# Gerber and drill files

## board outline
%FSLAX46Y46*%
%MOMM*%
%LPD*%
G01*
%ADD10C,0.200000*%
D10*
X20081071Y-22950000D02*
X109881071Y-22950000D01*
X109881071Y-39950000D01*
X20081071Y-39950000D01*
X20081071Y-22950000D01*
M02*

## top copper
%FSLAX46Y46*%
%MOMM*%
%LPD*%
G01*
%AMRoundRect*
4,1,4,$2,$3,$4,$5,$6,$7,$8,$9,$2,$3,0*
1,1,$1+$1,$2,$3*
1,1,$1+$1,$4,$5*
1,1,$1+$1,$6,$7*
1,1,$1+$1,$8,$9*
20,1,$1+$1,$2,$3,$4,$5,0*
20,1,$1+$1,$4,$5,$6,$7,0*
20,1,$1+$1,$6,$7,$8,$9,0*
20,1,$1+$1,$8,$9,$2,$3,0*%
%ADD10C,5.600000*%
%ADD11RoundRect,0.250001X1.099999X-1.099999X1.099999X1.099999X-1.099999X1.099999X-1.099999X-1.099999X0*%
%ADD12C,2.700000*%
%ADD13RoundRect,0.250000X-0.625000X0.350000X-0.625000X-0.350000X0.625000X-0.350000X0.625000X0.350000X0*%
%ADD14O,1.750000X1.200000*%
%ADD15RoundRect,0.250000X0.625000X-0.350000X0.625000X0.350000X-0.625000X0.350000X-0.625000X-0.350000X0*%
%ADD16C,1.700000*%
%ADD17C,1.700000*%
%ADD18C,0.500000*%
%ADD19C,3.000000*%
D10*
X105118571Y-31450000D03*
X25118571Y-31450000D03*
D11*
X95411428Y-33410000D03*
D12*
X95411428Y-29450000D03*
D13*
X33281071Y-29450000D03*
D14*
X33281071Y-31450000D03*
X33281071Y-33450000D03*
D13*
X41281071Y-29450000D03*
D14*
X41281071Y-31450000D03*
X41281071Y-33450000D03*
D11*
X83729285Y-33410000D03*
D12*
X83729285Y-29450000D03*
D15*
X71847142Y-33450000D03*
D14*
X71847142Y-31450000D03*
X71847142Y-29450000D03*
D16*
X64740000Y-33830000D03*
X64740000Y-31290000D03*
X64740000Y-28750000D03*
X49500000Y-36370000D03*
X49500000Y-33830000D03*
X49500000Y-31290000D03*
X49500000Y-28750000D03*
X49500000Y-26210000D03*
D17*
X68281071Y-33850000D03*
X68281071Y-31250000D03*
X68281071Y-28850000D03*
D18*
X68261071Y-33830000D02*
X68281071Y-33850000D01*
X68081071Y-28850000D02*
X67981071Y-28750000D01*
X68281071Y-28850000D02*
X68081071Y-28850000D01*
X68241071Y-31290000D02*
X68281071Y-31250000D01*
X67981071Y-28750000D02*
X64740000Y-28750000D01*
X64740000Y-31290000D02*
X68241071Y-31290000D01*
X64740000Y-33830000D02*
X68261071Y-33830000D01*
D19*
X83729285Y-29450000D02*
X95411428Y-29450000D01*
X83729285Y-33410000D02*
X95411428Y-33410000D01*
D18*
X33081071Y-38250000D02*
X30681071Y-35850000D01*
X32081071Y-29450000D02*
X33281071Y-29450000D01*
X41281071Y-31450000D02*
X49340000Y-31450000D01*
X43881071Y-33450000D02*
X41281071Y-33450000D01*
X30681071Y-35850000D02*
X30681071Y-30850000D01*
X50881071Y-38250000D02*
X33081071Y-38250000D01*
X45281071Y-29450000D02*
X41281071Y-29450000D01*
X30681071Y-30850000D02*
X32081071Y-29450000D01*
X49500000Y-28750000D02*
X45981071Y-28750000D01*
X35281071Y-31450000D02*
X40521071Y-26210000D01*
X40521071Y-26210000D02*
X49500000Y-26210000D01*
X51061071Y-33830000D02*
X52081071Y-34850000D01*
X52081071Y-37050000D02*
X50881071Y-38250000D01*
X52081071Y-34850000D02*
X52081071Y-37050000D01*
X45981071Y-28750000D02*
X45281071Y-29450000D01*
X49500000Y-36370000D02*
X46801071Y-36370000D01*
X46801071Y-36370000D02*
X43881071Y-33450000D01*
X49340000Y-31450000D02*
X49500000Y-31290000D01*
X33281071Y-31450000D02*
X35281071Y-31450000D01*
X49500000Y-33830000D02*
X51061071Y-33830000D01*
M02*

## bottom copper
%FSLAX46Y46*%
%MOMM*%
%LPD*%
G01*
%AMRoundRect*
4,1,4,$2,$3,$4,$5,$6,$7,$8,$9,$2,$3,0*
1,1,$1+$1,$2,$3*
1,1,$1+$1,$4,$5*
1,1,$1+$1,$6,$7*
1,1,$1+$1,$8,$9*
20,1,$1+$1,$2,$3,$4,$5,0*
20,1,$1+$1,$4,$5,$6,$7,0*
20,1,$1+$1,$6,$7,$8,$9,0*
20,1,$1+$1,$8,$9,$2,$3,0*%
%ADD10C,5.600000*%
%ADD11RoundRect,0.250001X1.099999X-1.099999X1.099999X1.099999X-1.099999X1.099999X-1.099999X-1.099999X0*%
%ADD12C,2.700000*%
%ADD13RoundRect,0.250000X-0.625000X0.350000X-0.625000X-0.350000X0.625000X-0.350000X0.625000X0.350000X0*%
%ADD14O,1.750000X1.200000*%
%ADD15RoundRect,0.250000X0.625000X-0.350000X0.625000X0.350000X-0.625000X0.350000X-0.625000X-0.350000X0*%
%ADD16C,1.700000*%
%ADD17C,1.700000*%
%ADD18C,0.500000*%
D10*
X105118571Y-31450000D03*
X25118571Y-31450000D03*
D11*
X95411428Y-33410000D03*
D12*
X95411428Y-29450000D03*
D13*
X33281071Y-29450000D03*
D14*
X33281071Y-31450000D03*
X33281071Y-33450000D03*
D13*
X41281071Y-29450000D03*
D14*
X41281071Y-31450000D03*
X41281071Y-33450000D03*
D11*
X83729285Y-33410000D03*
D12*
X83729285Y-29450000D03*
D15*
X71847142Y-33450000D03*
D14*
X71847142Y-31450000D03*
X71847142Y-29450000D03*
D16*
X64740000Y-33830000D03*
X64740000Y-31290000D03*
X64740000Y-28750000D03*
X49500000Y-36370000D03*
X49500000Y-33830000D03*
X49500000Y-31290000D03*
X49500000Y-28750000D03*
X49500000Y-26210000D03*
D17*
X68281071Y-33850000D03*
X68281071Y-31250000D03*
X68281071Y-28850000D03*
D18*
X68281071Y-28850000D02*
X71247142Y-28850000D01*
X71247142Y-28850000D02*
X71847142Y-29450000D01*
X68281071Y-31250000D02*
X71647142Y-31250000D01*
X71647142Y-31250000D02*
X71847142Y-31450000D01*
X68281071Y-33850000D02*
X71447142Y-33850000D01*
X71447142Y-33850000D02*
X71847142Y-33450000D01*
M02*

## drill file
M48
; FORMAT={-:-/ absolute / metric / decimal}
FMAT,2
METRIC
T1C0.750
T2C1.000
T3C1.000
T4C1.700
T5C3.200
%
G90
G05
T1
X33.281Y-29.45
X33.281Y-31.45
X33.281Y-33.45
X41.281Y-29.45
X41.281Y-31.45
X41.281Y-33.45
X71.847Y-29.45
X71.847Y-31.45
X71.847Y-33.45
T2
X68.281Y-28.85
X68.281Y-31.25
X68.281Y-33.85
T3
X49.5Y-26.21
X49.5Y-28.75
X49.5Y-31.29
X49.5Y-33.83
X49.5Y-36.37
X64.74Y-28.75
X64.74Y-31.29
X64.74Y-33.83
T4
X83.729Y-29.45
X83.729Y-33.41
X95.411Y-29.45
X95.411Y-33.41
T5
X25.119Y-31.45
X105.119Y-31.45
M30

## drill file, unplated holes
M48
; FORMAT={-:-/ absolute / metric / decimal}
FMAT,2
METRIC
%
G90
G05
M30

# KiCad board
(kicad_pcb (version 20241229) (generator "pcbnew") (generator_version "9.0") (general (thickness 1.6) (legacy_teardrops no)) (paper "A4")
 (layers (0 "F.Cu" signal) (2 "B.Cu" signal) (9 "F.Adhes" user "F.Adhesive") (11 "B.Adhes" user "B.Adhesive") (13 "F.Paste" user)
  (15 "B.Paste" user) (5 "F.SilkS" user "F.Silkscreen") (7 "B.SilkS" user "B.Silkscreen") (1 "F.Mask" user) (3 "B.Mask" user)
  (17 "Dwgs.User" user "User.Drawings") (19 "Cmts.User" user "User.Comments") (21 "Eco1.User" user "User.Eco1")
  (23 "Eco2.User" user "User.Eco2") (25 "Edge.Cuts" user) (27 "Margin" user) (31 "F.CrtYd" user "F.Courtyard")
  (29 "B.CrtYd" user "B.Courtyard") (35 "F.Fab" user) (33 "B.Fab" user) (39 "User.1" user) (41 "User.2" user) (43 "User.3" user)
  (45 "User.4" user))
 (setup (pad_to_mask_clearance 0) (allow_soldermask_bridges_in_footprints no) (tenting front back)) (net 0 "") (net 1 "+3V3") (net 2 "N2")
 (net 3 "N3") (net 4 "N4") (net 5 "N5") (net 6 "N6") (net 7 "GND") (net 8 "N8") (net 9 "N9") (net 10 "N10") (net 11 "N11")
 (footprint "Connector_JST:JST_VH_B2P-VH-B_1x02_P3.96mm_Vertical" (layer "F.Cu") (at 95.411428 33.41 90)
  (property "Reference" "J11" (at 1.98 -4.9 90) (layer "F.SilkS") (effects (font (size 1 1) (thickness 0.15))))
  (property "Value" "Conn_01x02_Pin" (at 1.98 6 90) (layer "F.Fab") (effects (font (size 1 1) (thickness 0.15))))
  (pad "1" thru_hole roundrect (at 0 0 90) (size 2.7 2.7) (drill 1.7) (layers "*.Cu" "*.Mask") (remove_unused_layers no)
   (roundrect_rratio 0.092593) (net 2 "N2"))
  (pad "2" thru_hole circle (at 3.96 0 90) (size 2.7 2.7) (drill 1.7) (layers "*.Cu" "*.Mask") (remove_unused_layers no) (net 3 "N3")))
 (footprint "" (layer "F.Cu") (at 105.118571 31.45)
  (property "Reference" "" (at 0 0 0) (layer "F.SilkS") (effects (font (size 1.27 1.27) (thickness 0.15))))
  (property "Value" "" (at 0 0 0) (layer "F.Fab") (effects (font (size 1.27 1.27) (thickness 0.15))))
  (pad "1" thru_hole circle (at 0 0) (size 5.6 5.6) (drill 3.2) (layers "*.Cu" "*.Mask") (remove_unused_layers no) (zone_connect 2)))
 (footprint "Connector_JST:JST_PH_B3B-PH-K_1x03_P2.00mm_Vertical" (layer "F.Cu") (at 71.847142 33.45 90)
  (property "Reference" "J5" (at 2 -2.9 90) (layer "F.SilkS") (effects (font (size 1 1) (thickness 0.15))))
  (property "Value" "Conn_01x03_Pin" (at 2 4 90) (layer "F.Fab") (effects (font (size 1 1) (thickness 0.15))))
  (pad "1" thru_hole roundrect (at 0 0 90) (size 1.2 1.75) (drill 0.75) (layers "*.Cu" "*.Mask") (remove_unused_layers no)
   (roundrect_rratio 0.208333) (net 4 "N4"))
  (pad "2" thru_hole oval (at 2 0 90) (size 1.2 1.75) (drill 0.75) (layers "*.Cu" "*.Mask") (remove_unused_layers no) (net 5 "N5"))
  (pad "3" thru_hole oval (at 4 0 90) (size 1.2 1.75) (drill 0.75) (layers "*.Cu" "*.Mask") (remove_unused_layers no) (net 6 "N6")))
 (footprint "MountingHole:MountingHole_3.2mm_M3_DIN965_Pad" (layer "F.Cu") (at 25.118571 31.45)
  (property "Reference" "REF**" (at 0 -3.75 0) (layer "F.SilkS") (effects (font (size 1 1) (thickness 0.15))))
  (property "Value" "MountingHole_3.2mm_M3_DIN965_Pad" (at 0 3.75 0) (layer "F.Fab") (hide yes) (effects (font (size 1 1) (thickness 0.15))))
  (pad "1" thru_hole circle (at 0 0) (size 5.6 5.6) (drill 3.2) (layers "*.Cu" "*.Mask") (remove_unused_layers no) (zone_connect 2)))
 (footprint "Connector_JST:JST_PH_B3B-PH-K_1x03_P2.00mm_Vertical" (layer "B.Cu") (at 33.281071 29.45 -90)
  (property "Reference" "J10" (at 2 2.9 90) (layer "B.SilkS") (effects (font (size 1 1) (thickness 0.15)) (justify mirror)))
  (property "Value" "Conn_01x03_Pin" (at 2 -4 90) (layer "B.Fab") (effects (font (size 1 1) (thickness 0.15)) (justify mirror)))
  (pad "1" thru_hole roundrect (at 0 0 270) (size 1.2 1.75) (drill 0.75) (layers "*.Cu" "*.Mask") (remove_unused_layers no)
   (roundrect_rratio 0.208333) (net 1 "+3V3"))
  (pad "2" thru_hole oval (at 2 0 270) (size 1.2 1.75) (drill 0.75) (layers "*.Cu" "*.Mask") (remove_unused_layers no) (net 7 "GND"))
  (pad "3" thru_hole oval (at 4 0 270) (size 1.2 1.75) (drill 0.75) (layers "*.Cu" "*.Mask") (remove_unused_layers no) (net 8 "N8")))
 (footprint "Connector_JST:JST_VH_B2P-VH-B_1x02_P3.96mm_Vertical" (layer "B.Cu") (at 83.729285 33.41 90)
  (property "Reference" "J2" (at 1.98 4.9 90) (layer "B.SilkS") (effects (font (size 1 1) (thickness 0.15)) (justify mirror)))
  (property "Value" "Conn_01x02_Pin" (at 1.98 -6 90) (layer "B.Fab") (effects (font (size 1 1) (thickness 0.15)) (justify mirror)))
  (pad "1" thru_hole roundrect (at 0 0 90) (size 2.7 2.7) (drill 1.7) (layers "*.Cu" "*.Mask") (remove_unused_layers no)
   (roundrect_rratio 0.092593) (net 2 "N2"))
  (pad "2" thru_hole circle (at 3.96 0 90) (size 2.7 2.7) (drill 1.7) (layers "*.Cu" "*.Mask") (remove_unused_layers no) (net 3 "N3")))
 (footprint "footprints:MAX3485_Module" (layer "B.Cu") (at 60.74 26.79 90)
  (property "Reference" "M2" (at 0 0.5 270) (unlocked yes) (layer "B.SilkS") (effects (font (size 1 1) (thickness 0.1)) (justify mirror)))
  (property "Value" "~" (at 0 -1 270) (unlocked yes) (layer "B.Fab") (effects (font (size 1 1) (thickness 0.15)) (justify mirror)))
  (pad "1" thru_hole circle (at -7.04 4 90) (size 1.7 1.7) (drill 1) (layers "*.Cu" "*.Mask") (remove_unused_layers no) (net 4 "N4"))
  (pad "2" thru_hole circle (at -4.5 4 90) (size 1.7 1.7) (drill 1) (layers "*.Cu" "*.Mask") (remove_unused_layers no) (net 5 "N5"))
  (pad "3" thru_hole circle (at -1.96 4 90) (size 1.7 1.7) (drill 1) (layers "*.Cu" "*.Mask") (remove_unused_layers no) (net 6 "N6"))
  (pad "4" thru_hole circle (at -9.58 -11.24 90) (size 1.7 1.7) (drill 1) (layers "*.Cu" "*.Mask") (remove_unused_layers no) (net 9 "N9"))
  (pad "5" thru_hole circle (at -7.04 -11.24 90) (size 1.7 1.7) (drill 1) (layers "*.Cu" "*.Mask") (remove_unused_layers no) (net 1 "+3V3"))
  (pad "6" thru_hole circle (at -4.5 -11.24 90) (size 1.7 1.7) (drill 1) (layers "*.Cu" "*.Mask") (remove_unused_layers no) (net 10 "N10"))
  (pad "7" thru_hole circle (at -1.96 -11.24 90) (size 1.7 1.7) (drill 1) (layers "*.Cu" "*.Mask") (remove_unused_layers no) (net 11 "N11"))
  (pad "8" thru_hole circle (at 0.58 -11.24 90) (size 1.7 1.7) (drill 1) (layers "*.Cu" "*.Mask") (remove_unused_layers no) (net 7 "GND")))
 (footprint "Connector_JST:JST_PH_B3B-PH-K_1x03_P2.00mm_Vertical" (layer "B.Cu") (at 41.281071 29.45 -90)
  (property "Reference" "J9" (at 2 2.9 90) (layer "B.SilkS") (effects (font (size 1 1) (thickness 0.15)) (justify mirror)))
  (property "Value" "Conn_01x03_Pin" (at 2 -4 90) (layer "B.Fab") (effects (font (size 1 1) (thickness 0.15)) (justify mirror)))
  (pad "1" thru_hole roundrect (at 0 0 270) (size 1.2 1.75) (drill 0.75) (layers "*.Cu" "*.Mask") (remove_unused_layers no)
   (roundrect_rratio 0.208333) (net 11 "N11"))
  (pad "2" thru_hole oval (at 2 0 270) (size 1.2 1.75) (drill 0.75) (layers "*.Cu" "*.Mask") (remove_unused_layers no) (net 10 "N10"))
  (pad "3" thru_hole oval (at 4 0 270) (size 1.2 1.75) (drill 0.75) (layers "*.Cu" "*.Mask") (remove_unused_layers no) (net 9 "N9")))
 (gr_rect (start 20.081071 22.95) (end 109.881071 39.95) (stroke (width 0.2) (type solid)) (fill no) (layer "Edge.Cuts"))
 (segment (start 52.081071 37.05) (end 50.881071 38.25) (width 0.5) (layer "F.Cu") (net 1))
 (segment (start 51.061071 33.83) (end 52.081071 34.85) (width 0.5) (layer "F.Cu") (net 1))
 (segment (start 32.081071 29.45) (end 33.281071 29.45) (width 0.5) (layer "F.Cu") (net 1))
 (segment (start 30.681071 30.85) (end 32.081071 29.45) (width 0.5) (layer "F.Cu") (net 1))
 (segment (start 30.681071 35.85) (end 30.681071 30.85) (width 0.5) (layer "F.Cu") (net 1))
 (segment (start 52.081071 34.85) (end 52.081071 37.05) (width 0.5) (layer "F.Cu") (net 1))
 (segment (start 33.081071 38.25) (end 30.681071 35.85) (width 0.5) (layer "F.Cu") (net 1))
 (segment (start 49.5 33.83) (end 51.061071 33.83) (width 0.5) (layer "F.Cu") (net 1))
 (segment (start 50.881071 38.25) (end 33.081071 38.25) (width 0.5) (layer "F.Cu") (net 1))
 (segment (start 40.521071 26.21) (end 49.5 26.21) (width 0.5) (layer "F.Cu") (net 7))
 (segment (start 35.281071 31.45) (end 40.521071 26.21) (width 0.5) (layer "F.Cu") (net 7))
 (segment (start 33.281071 31.45) (end 35.281071 31.45) (width 0.5) (layer "F.Cu") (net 7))
 (segment (start 41.281071 31.45) (end 49.34 31.45) (width 0.5) (layer "F.Cu") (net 10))
 (segment (start 49.34 31.45) (end 49.5 31.29) (width 0.5) (layer "F.Cu") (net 10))
 (segment (start 43.881071 33.45) (end 41.281071 33.45) (width 0.5) (layer "F.Cu") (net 9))
 (segment (start 46.801071 36.37) (end 43.881071 33.45) (width 0.5) (layer "F.Cu") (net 9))
 (segment (start 49.5 36.37) (end 46.801071 36.37) (width 0.5) (layer "F.Cu") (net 9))
 (segment (start 45.981071 28.75) (end 45.281071 29.45) (width 0.5) (layer "F.Cu") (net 11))
 (segment (start 49.5 28.75) (end 45.981071 28.75) (width 0.5) (layer "F.Cu") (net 11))
 (segment (start 45.281071 29.45) (end 41.281071 29.45) (width 0.5) (layer "F.Cu") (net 11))
 (segment (start 67.981071 28.75) (end 64.74 28.75) (width 0.5) (layer "F.Cu") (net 6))
 (segment (start 68.081071 28.85) (end 67.981071 28.75) (width 0.5) (layer "F.Cu") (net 6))
 (segment (start 68.281071 28.85) (end 68.081071 28.85) (width 0.5) (layer "F.Cu") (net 6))
 (via (at 68.281071 28.85) (size 1.7) (drill 1) (layers "F.Cu" "B.Cu") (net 6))
 (segment (start 68.281071 28.85) (end 71.247142 28.85) (width 0.5) (layer "B.Cu") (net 6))
 (segment (start 71.247142 28.85) (end 71.847142 29.45) (width 0.5) (layer "B.Cu") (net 6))
 (segment (start 68.241071 31.29) (end 68.281071 31.25) (width 0.5) (layer "F.Cu") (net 5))
 (segment (start 64.74 31.29) (end 68.241071 31.29) (width 0.5) (layer "F.Cu") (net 5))
 (via (at 68.281071 31.25) (size 1.7) (drill 1) (layers "F.Cu" "B.Cu") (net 5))
 (segment (start 71.647142 31.25) (end 71.847142 31.45) (width 0.5) (layer "B.Cu") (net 5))
 (segment (start 68.281071 31.25) (end 71.647142 31.25) (width 0.5) (layer "B.Cu") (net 5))
 (segment (start 68.261071 33.83) (end 68.281071 33.85) (width 0.5) (layer "F.Cu") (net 4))
 (segment (start 64.74 33.83) (end 68.261071 33.83) (width 0.5) (layer "F.Cu") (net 4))
 (via (at 68.281071 33.85) (size 1.7) (drill 1) (layers "F.Cu" "B.Cu") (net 4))
 (segment (start 71.447142 33.85) (end 71.847142 33.45) (width 0.5) (layer "B.Cu") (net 4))
 (segment (start 68.281071 33.85) (end 71.447142 33.85) (width 0.5) (layer "B.Cu") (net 4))
 (segment (start 83.729285 33.41) (end 95.411428 33.41) (width 3) (layer "F.Cu") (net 2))
 (segment (start 83.729285 29.45) (end 95.411428 29.45) (width 3) (layer "F.Cu") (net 3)))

